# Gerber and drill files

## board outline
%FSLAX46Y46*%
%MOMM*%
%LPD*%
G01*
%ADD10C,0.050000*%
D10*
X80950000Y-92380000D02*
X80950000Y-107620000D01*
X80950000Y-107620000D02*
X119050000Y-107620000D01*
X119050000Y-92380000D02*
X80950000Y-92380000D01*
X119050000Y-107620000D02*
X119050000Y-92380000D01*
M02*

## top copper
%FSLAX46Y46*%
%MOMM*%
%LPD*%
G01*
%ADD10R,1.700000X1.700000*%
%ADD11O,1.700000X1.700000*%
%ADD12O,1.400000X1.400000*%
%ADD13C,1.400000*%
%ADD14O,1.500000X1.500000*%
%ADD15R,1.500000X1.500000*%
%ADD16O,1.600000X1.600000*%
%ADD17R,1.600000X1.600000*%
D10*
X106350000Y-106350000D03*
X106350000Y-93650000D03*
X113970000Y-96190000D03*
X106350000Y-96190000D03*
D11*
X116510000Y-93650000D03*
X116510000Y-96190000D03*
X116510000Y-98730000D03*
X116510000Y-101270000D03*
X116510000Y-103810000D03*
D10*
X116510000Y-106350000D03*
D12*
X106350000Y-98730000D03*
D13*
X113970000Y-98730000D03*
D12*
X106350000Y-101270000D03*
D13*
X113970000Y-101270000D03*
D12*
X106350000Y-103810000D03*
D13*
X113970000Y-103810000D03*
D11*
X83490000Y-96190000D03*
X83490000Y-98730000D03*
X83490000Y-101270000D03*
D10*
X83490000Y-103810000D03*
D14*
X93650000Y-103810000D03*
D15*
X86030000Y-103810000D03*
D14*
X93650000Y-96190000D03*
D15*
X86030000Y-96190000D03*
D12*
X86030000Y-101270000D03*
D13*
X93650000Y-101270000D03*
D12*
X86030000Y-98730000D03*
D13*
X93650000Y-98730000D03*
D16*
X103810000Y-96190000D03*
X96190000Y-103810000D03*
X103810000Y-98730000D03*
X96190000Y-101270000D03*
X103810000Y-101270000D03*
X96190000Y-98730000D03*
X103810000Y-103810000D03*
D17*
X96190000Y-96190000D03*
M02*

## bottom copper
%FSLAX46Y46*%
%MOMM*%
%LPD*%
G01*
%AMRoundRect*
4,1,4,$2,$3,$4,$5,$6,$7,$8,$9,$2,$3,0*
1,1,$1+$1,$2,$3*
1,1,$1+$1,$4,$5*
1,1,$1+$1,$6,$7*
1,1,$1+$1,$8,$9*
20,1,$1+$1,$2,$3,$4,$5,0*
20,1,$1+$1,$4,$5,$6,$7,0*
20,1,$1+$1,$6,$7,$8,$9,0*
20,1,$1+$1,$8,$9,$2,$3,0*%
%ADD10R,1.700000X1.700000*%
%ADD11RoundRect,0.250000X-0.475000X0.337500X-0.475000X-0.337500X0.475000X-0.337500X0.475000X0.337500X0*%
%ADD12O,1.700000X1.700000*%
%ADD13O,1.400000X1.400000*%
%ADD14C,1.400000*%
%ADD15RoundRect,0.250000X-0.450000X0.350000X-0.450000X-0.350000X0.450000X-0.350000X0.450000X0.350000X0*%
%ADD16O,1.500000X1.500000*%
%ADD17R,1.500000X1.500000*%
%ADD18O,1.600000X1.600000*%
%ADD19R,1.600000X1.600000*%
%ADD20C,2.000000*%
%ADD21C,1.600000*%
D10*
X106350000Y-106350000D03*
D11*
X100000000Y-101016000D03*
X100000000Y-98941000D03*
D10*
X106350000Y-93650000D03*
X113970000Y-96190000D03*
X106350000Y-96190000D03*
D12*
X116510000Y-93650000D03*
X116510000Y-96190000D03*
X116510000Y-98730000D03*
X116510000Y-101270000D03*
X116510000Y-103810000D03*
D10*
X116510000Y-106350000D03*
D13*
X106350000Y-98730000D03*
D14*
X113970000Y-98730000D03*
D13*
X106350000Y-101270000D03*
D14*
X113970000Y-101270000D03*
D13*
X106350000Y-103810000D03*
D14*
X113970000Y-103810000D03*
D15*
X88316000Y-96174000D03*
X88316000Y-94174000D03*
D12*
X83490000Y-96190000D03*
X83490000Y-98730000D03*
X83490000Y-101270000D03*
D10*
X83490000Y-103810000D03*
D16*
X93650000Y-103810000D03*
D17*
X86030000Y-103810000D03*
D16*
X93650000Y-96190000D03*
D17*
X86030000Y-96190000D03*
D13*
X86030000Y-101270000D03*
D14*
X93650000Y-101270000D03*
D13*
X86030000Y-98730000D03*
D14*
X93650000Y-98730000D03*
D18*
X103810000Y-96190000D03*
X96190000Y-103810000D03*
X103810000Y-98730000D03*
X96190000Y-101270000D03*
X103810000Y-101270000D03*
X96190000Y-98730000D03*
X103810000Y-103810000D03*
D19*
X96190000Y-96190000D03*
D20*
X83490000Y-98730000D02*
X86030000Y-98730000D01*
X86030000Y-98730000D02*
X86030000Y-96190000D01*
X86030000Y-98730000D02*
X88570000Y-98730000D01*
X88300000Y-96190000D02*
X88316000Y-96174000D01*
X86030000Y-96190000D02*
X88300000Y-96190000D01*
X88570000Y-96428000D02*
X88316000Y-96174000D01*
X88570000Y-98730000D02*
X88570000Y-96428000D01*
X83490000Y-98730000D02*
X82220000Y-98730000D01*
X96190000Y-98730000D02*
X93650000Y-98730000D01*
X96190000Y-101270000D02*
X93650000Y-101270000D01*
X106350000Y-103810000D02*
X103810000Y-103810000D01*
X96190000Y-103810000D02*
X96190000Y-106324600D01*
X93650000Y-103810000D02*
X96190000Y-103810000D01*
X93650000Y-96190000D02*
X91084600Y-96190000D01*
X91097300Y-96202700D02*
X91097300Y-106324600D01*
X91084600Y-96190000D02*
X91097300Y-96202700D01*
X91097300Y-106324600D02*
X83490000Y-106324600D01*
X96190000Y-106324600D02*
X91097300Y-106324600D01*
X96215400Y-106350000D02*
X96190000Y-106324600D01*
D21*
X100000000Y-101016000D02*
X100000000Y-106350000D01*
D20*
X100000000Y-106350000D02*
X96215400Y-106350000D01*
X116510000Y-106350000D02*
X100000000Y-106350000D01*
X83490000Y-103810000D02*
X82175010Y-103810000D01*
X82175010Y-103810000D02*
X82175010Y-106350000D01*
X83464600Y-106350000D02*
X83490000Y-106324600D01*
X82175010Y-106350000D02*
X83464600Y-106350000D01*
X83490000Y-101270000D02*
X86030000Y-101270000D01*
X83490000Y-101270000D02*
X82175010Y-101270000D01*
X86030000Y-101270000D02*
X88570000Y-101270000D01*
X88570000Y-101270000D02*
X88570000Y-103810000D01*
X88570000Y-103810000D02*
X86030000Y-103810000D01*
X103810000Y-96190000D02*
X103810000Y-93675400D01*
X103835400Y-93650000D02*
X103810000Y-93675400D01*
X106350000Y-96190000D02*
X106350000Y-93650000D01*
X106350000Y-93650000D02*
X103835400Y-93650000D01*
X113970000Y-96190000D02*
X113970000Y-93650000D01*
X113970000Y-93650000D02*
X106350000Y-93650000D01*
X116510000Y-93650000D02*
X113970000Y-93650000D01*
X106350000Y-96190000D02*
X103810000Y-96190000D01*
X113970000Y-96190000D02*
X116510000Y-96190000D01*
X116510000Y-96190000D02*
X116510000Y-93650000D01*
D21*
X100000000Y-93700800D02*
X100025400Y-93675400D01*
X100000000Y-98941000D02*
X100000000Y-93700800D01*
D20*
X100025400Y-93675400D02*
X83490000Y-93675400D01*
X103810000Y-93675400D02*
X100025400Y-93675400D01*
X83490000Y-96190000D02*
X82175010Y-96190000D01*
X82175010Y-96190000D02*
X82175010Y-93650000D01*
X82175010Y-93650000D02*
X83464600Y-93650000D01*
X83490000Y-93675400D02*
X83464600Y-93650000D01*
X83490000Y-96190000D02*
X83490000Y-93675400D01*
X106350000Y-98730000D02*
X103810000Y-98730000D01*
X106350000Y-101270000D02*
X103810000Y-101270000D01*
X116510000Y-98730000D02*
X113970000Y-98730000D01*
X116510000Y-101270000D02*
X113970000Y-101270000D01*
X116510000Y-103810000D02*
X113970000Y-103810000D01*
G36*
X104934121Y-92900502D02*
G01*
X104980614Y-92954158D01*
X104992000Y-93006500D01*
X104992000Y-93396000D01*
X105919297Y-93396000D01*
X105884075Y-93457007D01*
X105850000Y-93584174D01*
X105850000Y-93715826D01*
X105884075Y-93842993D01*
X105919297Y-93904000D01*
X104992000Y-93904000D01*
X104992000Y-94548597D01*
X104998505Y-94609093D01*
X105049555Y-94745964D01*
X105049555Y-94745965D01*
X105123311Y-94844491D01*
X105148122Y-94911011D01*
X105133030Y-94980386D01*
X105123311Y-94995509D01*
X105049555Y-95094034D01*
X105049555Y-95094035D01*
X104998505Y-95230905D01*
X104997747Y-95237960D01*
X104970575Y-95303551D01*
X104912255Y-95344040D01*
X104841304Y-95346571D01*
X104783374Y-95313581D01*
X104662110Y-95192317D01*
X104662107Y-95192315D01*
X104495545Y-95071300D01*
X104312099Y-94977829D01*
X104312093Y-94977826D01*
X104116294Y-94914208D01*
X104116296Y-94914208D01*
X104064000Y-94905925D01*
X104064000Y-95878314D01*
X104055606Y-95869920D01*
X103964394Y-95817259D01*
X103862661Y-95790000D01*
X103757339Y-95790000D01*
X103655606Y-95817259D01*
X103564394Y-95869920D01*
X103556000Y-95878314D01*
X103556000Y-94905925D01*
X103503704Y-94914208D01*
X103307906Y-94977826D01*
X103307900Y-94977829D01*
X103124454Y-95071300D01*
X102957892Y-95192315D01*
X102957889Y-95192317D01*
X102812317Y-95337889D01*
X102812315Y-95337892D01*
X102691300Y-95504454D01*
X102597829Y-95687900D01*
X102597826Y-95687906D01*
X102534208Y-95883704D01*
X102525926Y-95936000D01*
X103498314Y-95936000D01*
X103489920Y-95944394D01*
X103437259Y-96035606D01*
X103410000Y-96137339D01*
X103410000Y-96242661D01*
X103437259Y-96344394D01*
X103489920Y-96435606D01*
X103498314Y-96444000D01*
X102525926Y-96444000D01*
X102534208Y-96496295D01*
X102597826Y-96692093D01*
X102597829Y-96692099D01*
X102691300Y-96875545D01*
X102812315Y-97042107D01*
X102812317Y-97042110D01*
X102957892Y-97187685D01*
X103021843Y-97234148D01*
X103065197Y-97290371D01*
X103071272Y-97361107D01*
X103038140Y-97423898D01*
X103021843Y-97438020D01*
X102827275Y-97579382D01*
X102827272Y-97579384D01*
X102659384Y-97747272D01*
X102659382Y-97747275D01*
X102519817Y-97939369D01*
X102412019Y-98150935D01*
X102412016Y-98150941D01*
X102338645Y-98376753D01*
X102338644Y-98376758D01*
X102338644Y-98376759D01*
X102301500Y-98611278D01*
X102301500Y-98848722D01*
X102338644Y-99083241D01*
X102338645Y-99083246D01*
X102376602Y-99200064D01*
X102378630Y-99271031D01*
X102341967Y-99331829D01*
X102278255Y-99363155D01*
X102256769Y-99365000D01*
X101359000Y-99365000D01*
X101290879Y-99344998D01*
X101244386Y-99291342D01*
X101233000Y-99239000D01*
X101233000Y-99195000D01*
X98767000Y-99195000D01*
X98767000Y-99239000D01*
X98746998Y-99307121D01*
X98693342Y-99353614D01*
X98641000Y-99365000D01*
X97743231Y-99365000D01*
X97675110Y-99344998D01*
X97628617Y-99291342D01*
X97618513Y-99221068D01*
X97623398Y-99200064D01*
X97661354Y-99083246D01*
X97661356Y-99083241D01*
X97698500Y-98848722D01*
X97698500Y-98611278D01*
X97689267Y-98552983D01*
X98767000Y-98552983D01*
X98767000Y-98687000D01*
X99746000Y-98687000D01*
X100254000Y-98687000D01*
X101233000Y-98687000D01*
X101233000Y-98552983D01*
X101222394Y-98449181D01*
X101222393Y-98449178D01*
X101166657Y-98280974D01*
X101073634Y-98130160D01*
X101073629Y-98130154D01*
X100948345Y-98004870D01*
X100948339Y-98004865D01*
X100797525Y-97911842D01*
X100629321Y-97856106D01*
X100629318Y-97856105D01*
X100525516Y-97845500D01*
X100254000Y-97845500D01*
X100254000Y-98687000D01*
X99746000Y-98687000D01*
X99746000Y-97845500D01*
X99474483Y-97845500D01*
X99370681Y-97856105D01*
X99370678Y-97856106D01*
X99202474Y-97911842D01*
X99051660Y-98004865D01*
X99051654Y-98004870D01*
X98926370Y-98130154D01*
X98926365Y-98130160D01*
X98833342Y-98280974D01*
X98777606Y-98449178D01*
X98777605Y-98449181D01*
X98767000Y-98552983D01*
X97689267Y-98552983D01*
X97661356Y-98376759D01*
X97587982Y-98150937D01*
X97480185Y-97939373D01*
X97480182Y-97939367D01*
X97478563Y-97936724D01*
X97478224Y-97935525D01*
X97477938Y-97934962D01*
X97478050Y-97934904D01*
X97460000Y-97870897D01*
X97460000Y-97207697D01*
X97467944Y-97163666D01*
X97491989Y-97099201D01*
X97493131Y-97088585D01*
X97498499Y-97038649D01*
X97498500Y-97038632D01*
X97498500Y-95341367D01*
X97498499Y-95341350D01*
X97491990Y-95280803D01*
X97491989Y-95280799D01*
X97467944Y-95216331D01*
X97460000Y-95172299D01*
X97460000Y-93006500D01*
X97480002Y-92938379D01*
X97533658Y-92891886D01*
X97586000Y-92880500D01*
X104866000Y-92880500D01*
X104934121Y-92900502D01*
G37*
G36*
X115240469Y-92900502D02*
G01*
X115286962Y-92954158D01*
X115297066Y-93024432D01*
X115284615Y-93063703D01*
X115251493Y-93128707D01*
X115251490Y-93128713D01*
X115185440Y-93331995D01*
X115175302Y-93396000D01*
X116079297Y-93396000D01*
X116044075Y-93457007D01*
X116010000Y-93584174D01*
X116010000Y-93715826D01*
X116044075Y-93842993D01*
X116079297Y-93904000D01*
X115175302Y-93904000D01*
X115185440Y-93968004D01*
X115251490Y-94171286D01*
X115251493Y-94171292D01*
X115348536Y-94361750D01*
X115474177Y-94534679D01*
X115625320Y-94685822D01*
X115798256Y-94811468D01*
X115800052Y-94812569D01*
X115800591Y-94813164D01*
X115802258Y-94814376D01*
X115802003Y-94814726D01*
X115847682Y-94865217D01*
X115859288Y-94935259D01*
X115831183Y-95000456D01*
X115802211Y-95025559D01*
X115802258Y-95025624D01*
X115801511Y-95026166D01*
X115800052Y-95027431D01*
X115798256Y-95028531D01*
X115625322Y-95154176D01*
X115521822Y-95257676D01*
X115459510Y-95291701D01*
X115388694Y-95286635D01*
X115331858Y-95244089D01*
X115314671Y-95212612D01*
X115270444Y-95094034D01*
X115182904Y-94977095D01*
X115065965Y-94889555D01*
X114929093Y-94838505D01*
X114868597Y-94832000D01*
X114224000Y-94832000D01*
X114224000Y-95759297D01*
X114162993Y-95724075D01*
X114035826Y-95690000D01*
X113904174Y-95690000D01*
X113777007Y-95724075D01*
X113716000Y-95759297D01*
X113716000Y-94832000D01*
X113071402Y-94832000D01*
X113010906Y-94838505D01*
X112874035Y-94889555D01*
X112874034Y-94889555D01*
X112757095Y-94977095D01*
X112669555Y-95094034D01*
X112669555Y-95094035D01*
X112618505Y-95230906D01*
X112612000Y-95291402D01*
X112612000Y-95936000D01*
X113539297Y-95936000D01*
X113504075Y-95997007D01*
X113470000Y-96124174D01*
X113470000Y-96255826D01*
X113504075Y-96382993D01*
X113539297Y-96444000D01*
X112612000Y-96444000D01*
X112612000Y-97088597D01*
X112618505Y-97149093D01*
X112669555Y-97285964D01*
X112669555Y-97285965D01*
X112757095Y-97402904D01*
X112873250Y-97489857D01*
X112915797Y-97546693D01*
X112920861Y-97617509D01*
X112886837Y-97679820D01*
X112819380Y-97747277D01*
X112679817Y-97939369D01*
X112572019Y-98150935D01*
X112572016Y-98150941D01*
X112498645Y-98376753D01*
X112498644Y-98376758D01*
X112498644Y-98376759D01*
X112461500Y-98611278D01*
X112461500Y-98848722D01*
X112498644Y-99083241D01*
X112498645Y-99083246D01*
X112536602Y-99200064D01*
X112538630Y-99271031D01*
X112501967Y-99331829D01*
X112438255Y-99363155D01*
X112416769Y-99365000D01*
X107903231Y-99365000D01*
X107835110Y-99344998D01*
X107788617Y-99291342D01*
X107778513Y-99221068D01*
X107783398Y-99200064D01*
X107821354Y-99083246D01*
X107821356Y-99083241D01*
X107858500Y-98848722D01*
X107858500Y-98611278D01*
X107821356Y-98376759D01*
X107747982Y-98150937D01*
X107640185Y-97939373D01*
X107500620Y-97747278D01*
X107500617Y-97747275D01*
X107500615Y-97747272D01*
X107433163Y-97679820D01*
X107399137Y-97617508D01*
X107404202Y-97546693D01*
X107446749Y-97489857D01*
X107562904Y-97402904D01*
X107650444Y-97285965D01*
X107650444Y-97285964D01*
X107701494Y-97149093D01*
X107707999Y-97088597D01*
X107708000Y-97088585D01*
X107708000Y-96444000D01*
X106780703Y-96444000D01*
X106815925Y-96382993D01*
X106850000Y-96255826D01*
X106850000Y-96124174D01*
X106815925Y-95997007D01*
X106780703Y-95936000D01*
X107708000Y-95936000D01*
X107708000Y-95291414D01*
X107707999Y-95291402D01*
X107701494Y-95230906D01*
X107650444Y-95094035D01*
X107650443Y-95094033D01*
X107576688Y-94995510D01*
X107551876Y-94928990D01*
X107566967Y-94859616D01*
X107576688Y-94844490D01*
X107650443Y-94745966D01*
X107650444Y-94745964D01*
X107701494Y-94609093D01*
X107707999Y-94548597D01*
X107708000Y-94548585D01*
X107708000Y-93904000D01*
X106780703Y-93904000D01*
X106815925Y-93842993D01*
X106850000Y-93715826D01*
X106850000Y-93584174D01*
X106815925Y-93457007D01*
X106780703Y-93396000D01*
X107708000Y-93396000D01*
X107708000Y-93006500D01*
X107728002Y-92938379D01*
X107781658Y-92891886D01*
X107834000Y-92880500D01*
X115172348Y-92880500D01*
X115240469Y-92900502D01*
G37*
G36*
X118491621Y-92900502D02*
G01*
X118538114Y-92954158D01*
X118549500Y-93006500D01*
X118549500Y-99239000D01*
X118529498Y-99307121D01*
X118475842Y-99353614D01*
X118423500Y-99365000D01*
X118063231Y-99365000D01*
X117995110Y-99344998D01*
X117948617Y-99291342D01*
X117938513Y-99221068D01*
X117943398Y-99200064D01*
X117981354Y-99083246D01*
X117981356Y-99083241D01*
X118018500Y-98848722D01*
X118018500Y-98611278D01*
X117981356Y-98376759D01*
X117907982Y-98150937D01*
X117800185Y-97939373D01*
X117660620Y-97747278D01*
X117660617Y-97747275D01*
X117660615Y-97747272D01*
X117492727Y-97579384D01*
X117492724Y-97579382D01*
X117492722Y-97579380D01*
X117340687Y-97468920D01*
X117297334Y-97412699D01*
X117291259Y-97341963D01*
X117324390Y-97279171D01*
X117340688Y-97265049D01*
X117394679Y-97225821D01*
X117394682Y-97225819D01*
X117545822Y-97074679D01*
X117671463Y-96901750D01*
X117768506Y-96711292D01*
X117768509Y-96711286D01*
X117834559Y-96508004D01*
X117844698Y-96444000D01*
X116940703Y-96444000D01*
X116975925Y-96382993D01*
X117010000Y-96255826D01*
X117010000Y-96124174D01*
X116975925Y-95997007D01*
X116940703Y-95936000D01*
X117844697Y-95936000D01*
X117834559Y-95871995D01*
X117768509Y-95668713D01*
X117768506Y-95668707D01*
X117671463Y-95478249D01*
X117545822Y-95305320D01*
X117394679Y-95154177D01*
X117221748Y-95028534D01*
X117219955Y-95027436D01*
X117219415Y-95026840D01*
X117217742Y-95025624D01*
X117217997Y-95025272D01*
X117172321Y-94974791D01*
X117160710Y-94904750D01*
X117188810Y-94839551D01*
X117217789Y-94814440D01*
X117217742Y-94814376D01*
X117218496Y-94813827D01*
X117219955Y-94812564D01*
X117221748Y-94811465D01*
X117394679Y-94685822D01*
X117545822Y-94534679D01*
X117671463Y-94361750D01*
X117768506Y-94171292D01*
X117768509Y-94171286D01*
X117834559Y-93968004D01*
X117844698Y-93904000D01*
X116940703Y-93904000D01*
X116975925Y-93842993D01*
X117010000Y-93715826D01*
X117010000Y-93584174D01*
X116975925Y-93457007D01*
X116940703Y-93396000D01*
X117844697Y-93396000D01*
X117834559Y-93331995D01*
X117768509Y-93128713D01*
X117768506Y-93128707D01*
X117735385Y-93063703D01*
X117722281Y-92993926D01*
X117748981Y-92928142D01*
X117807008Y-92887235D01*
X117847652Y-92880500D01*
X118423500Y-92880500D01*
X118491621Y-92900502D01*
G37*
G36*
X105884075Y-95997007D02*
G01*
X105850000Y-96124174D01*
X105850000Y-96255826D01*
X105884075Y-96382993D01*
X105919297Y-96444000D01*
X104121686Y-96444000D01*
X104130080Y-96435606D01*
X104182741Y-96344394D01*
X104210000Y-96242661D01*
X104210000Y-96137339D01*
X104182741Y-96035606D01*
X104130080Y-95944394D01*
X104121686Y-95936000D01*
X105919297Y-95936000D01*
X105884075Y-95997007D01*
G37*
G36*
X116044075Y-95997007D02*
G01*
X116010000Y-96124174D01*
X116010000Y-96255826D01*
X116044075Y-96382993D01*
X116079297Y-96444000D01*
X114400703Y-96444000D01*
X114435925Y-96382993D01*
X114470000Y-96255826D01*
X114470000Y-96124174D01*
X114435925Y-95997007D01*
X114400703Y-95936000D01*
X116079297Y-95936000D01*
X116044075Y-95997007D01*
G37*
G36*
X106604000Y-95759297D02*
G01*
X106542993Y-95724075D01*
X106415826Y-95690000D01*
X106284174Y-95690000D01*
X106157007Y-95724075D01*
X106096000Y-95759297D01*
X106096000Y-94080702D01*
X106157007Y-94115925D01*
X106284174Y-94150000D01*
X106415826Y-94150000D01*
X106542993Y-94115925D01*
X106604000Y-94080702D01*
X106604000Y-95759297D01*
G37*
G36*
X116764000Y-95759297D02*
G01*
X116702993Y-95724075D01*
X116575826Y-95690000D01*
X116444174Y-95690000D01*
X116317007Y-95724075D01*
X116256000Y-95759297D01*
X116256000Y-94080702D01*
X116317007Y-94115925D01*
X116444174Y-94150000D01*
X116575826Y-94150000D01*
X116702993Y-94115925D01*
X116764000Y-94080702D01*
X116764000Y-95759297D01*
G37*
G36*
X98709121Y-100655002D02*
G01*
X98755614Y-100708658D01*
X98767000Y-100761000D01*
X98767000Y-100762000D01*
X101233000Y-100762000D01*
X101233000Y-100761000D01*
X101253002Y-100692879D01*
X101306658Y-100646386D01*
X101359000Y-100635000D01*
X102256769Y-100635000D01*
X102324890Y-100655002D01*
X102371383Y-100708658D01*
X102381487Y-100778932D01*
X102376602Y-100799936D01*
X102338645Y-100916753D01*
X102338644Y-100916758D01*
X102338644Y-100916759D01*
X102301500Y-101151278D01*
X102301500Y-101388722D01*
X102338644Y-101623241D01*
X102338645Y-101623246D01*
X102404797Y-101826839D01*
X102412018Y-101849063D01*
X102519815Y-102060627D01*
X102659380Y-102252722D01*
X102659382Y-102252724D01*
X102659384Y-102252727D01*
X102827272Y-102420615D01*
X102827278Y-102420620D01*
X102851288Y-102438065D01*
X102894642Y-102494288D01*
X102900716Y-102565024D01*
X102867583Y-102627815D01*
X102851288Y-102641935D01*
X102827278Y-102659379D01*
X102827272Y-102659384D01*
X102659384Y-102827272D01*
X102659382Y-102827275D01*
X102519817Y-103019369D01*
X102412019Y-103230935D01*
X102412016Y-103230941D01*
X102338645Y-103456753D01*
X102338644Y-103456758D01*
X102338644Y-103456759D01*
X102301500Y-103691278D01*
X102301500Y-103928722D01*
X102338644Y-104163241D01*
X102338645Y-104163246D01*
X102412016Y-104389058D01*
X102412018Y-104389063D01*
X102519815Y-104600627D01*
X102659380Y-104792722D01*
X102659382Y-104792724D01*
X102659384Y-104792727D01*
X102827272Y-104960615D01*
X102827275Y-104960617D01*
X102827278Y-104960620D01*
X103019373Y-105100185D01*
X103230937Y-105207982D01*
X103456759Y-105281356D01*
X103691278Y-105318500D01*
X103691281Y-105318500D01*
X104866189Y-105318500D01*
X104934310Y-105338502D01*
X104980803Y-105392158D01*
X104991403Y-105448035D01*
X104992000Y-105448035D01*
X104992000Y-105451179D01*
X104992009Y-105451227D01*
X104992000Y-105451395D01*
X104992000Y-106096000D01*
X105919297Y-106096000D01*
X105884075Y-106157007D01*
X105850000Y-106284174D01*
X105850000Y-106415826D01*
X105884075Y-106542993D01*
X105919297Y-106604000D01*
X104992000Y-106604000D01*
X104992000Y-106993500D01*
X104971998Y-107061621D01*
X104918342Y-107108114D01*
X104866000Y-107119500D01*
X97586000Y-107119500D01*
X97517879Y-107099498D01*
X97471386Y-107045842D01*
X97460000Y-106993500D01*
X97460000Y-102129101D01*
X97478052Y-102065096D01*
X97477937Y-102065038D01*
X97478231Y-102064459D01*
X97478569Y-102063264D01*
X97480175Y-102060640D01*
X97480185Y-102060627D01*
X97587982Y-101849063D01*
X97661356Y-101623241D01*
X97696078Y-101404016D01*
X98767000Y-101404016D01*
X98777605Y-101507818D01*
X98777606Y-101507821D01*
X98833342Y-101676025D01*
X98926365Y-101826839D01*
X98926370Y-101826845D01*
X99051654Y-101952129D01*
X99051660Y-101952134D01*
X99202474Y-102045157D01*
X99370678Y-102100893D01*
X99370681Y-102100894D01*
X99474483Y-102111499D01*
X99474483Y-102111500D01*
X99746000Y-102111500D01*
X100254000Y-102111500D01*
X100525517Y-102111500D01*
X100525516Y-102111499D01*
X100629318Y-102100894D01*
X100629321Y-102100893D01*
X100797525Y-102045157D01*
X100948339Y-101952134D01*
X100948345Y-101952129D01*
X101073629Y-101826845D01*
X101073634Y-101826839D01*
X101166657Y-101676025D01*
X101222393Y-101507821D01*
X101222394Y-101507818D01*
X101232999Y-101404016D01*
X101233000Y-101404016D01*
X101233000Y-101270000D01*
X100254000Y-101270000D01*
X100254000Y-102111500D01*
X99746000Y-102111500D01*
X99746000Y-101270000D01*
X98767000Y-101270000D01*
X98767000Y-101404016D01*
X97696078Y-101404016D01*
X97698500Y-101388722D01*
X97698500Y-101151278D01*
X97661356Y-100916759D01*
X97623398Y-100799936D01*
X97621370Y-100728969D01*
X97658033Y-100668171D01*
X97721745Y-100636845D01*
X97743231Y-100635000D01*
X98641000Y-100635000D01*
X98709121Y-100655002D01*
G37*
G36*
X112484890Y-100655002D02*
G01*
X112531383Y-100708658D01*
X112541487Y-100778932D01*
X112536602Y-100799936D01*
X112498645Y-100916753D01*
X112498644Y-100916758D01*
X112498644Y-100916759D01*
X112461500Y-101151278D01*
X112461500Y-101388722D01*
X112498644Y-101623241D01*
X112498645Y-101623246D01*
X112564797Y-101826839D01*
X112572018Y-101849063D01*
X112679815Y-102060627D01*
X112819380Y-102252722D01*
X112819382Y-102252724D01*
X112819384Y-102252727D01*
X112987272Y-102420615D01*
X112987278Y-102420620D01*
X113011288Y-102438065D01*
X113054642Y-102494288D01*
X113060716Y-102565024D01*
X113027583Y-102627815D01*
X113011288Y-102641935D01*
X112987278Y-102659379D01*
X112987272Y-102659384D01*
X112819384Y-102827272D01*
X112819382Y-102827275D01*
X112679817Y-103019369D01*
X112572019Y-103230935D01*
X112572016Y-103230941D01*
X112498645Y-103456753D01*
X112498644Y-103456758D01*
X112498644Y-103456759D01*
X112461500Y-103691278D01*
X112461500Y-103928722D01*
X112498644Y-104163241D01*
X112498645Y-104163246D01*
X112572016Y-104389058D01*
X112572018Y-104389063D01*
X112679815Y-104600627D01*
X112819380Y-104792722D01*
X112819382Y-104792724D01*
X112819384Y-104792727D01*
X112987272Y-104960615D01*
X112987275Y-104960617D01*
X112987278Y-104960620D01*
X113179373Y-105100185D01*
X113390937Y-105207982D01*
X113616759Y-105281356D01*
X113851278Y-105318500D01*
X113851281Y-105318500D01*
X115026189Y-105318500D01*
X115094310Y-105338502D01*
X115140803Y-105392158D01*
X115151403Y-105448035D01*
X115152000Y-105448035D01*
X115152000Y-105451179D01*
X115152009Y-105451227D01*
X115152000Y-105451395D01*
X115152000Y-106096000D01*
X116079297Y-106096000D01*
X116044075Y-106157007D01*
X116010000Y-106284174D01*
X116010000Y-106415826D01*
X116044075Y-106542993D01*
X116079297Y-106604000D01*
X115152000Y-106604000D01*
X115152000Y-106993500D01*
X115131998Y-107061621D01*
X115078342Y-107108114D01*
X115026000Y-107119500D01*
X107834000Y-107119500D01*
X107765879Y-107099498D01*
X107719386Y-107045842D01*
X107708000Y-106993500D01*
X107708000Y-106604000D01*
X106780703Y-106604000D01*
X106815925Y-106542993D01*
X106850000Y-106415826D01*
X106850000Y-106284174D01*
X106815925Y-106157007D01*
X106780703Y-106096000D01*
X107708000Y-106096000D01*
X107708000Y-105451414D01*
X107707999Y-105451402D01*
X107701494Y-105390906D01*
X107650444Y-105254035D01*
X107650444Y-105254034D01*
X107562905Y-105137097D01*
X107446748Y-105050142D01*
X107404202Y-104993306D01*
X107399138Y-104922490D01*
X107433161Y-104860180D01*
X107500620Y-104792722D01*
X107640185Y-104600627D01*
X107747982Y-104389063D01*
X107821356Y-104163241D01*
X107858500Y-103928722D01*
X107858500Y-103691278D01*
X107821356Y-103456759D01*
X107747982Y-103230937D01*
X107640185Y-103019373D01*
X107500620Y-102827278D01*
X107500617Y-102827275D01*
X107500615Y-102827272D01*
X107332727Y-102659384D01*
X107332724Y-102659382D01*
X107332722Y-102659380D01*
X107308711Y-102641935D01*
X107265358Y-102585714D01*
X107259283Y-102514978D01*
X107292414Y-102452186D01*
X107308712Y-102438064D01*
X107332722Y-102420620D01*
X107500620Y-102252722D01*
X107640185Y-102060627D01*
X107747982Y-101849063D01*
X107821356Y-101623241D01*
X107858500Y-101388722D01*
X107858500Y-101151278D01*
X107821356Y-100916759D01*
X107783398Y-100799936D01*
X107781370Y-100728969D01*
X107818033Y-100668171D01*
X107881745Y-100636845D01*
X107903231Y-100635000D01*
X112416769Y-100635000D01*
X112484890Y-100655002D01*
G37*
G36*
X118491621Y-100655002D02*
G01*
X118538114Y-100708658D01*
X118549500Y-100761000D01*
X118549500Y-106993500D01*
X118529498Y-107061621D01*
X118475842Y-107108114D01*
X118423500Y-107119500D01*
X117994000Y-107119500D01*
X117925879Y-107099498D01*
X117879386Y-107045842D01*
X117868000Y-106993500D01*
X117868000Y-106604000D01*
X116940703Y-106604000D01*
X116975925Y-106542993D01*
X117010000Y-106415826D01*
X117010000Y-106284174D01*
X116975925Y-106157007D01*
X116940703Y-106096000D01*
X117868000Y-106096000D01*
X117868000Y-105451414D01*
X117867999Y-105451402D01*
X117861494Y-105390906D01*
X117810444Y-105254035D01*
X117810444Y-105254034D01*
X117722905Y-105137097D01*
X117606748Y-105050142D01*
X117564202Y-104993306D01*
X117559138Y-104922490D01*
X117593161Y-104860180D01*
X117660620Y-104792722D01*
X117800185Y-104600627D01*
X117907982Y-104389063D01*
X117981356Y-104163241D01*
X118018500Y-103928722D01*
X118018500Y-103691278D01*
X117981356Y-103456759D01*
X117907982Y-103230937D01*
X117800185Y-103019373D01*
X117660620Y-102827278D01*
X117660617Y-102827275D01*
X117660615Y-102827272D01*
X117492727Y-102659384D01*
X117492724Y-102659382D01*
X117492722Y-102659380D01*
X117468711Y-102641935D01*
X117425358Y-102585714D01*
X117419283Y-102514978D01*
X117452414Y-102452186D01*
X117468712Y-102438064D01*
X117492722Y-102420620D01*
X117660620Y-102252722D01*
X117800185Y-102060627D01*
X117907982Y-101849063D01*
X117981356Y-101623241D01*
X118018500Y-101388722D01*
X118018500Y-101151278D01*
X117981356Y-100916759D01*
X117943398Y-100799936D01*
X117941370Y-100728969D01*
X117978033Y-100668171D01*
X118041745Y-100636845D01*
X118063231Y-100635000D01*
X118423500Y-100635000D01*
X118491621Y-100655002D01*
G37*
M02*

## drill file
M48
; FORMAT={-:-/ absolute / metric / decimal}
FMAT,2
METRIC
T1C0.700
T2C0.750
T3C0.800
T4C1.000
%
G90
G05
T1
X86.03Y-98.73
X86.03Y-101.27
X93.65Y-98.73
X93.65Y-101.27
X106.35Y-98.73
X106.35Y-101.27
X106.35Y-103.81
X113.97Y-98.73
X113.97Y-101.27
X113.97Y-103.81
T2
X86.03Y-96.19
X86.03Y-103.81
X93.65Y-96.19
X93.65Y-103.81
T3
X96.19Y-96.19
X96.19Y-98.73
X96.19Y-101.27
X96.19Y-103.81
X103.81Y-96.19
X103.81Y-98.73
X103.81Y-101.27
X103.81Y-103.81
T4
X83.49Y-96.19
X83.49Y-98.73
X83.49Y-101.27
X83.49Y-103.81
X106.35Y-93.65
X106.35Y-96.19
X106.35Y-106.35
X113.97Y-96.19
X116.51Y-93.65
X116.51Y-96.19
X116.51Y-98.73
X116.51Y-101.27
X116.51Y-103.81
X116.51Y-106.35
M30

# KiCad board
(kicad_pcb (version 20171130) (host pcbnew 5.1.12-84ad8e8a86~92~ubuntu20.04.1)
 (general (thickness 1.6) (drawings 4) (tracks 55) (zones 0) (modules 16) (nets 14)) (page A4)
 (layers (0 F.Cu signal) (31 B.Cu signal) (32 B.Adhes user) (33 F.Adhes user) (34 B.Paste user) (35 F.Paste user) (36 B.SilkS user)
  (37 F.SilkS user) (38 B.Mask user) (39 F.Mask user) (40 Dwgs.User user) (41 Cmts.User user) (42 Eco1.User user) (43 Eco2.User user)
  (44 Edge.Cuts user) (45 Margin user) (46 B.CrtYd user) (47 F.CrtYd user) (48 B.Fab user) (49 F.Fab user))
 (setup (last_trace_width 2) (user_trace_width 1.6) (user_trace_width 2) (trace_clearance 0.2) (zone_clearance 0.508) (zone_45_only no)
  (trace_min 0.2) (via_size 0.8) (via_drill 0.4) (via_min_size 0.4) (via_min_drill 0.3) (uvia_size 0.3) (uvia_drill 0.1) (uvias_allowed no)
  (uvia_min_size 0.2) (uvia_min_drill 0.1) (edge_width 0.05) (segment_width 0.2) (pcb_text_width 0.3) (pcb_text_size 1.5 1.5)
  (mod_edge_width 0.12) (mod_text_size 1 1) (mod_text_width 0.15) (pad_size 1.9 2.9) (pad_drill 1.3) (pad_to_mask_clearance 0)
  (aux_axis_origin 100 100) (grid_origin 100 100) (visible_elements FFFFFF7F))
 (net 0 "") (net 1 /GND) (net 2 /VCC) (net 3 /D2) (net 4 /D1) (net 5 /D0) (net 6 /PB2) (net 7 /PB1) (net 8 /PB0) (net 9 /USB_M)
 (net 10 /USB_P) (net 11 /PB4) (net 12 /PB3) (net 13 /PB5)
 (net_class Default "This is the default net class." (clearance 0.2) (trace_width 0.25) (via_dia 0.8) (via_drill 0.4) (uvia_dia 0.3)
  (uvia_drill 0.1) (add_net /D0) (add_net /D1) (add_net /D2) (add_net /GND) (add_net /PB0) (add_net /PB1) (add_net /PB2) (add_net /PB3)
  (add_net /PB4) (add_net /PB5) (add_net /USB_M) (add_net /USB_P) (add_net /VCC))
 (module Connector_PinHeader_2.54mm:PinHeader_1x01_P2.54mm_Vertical (layer F.Cu) (at 106.35 106.35)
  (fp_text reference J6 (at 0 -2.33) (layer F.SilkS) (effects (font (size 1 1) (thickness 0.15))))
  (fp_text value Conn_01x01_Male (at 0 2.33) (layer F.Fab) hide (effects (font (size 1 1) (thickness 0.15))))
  (pad 1 thru_hole rect (at 0 0) (size 1.7 1.7) (drill 1) (layers *.Cu *.Mask) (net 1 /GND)))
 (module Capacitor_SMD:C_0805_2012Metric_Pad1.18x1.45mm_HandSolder (layer B.Cu) (at 100 99.9785 270)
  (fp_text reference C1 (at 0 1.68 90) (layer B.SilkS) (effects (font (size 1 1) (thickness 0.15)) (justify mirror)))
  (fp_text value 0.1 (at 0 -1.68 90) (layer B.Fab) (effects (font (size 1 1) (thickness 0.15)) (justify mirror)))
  (pad 2 smd roundrect (at 1.0375 0 270) (size 1.175 1.45) (layers B.Cu B.Paste B.Mask) (roundrect_rratio 0.212766) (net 1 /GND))
  (pad 1 smd roundrect (at -1.0375 0 270) (size 1.175 1.45) (layers B.Cu B.Paste B.Mask) (roundrect_rratio 0.212766) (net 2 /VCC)))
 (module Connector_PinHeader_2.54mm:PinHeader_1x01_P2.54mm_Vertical (layer F.Cu) (at 106.35 93.65)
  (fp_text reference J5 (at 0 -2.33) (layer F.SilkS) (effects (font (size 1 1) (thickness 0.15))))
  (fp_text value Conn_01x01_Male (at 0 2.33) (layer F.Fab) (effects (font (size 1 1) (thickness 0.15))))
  (pad 1 thru_hole rect (at 0 0) (size 1.7 1.7) (drill 1) (layers *.Cu *.Mask) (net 2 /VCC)))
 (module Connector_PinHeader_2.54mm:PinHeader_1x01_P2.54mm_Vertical (layer F.Cu) (at 113.97 96.19)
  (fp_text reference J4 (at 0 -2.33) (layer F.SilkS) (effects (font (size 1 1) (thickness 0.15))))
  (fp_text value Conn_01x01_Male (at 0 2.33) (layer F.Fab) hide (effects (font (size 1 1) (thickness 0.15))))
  (pad 1 thru_hole rect (at 0 0) (size 1.7 1.7) (drill 1) (layers *.Cu *.Mask) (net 2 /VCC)))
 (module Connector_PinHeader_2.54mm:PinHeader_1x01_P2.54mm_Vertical (layer F.Cu) (at 106.35 96.19)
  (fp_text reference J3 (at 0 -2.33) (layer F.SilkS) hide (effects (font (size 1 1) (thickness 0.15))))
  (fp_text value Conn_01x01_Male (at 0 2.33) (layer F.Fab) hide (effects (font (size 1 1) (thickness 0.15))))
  (pad 1 thru_hole rect (at 0 0) (size 1.7 1.7) (drill 1) (layers *.Cu *.Mask) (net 2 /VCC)))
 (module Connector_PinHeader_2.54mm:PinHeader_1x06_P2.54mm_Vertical (layer F.Cu) (at 116.51 106.35 180)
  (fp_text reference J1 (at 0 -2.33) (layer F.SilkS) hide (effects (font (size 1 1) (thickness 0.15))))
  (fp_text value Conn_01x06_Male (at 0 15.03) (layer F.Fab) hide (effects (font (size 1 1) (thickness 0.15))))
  (pad 6 thru_hole oval (at 0 12.7 180) (size 1.7 1.7) (drill 1) (layers *.Cu *.Mask) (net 2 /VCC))
  (pad 5 thru_hole oval (at 0 10.16 180) (size 1.7 1.7) (drill 1) (layers *.Cu *.Mask) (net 2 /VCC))
  (pad 4 thru_hole oval (at 0 7.62 180) (size 1.7 1.7) (drill 1) (layers *.Cu *.Mask) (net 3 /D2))
  (pad 3 thru_hole oval (at 0 5.08 180) (size 1.7 1.7) (drill 1) (layers *.Cu *.Mask) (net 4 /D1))
  (pad 2 thru_hole oval (at 0 2.54 180) (size 1.7 1.7) (drill 1) (layers *.Cu *.Mask) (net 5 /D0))
  (pad 1 thru_hole rect (at 0 0 180) (size 1.7 1.7) (drill 1) (layers *.Cu *.Mask) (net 1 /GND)))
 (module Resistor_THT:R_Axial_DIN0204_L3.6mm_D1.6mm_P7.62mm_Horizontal (layer F.Cu) (at 113.97 98.73 180)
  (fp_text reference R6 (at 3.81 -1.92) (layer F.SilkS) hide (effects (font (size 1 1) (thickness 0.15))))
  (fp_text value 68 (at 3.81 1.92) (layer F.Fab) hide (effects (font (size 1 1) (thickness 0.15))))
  (pad 2 thru_hole oval (at 7.62 0 180) (size 1.4 1.4) (drill 0.7) (layers *.Cu *.Mask) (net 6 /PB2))
  (pad 1 thru_hole circle (at 0 0 180) (size 1.4 1.4) (drill 0.7) (layers *.Cu *.Mask) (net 3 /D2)))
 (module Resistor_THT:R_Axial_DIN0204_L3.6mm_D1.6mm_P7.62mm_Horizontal (layer F.Cu) (at 113.97 101.27 180)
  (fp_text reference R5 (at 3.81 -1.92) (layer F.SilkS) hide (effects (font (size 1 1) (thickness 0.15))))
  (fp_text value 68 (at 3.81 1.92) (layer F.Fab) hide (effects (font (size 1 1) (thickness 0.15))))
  (pad 2 thru_hole oval (at 7.62 0 180) (size 1.4 1.4) (drill 0.7) (layers *.Cu *.Mask) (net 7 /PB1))
  (pad 1 thru_hole circle (at 0 0 180) (size 1.4 1.4) (drill 0.7) (layers *.Cu *.Mask) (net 4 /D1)))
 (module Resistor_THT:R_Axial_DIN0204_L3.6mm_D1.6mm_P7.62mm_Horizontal (layer F.Cu) (at 113.97 103.81 180)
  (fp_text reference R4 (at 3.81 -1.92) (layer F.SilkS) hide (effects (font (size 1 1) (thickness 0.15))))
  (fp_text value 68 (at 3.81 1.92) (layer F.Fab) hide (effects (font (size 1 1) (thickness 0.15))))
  (pad 2 thru_hole oval (at 7.62 0 180) (size 1.4 1.4) (drill 0.7) (layers *.Cu *.Mask) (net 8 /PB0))
  (pad 1 thru_hole circle (at 0 0 180) (size 1.4 1.4) (drill 0.7) (layers *.Cu *.Mask) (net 5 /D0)))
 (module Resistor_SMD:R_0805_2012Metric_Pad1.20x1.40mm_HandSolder (layer B.Cu) (at 88.316 95.174 270)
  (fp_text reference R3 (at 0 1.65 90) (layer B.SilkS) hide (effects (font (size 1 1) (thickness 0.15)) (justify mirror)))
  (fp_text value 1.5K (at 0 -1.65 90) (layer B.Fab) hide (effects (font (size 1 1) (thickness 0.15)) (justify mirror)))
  (pad 2 smd roundrect (at 1 0 270) (size 1.2 1.4) (layers B.Cu B.Paste B.Mask) (roundrect_rratio 0.208333) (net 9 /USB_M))
  (pad 1 smd roundrect (at -1 0 270) (size 1.2 1.4) (layers B.Cu B.Paste B.Mask) (roundrect_rratio 0.208333) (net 2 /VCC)))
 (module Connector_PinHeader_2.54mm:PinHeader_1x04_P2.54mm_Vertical (layer F.Cu) (at 83.49 103.81 180)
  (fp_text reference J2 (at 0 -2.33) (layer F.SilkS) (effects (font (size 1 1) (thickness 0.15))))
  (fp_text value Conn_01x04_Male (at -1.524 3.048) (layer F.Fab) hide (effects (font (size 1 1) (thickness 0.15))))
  (pad 4 thru_hole oval (at 0 7.62 180) (size 1.7 1.7) (drill 1) (layers *.Cu *.Mask) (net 2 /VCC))
  (pad 3 thru_hole oval (at 0 5.08 180) (size 1.7 1.7) (drill 1) (layers *.Cu *.Mask) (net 9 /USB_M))
  (pad 2 thru_hole oval (at 0 2.54 180) (size 1.7 1.7) (drill 1) (layers *.Cu *.Mask) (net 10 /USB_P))
  (pad 1 thru_hole rect (at 0 0 180) (size 1.7 1.7) (drill 1) (layers *.Cu *.Mask) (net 1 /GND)))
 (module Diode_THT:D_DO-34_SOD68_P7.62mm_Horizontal (layer F.Cu) (at 86.03 103.81)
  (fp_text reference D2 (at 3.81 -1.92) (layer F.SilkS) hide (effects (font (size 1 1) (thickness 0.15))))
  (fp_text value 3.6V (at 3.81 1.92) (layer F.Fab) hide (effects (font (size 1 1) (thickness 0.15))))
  (pad 2 thru_hole oval (at 7.62 0) (size 1.5 1.5) (drill 0.75) (layers *.Cu *.Mask) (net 1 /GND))
  (pad 1 thru_hole rect (at 0 0) (size 1.5 1.5) (drill 0.75) (layers *.Cu *.Mask) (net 10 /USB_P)))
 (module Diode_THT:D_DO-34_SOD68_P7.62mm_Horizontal (layer F.Cu) (at 86.03 96.19)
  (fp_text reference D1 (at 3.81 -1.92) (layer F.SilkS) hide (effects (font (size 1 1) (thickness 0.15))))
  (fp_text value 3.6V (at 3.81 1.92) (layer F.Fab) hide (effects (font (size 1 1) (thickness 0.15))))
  (pad 2 thru_hole oval (at 7.62 0) (size 1.5 1.5) (drill 0.75) (layers *.Cu *.Mask) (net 1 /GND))
  (pad 1 thru_hole rect (at 0 0) (size 1.5 1.5) (drill 0.75) (layers *.Cu *.Mask) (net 9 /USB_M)))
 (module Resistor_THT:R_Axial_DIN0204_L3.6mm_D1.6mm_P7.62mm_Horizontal (layer F.Cu) (at 93.65 101.27 180)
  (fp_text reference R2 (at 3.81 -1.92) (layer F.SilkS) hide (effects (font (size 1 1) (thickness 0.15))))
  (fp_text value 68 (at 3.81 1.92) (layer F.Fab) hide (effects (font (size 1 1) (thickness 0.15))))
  (pad 2 thru_hole oval (at 7.62 0 180) (size 1.4 1.4) (drill 0.7) (layers *.Cu *.Mask) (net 10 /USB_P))
  (pad 1 thru_hole circle (at 0 0 180) (size 1.4 1.4) (drill 0.7) (layers *.Cu *.Mask) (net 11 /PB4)))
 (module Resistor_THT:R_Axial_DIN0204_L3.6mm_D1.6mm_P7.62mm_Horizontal (layer F.Cu) (at 93.65 98.73 180)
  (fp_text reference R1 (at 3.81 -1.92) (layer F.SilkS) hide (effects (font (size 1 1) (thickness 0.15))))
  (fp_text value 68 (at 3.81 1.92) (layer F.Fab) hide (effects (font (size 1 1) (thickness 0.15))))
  (pad 2 thru_hole oval (at 7.62 0 180) (size 1.4 1.4) (drill 0.7) (layers *.Cu *.Mask) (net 9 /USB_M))
  (pad 1 thru_hole circle (at 0 0 180) (size 1.4 1.4) (drill 0.7) (layers *.Cu *.Mask) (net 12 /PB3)))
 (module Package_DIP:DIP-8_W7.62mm (layer F.Cu) (at 96.19 96.19)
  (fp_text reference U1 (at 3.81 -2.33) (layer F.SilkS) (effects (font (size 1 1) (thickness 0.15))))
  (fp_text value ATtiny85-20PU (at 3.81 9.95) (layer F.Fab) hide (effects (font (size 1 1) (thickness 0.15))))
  (pad 8 thru_hole oval (at 7.62 0) (size 1.6 1.6) (drill 0.8) (layers *.Cu *.Mask) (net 2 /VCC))
  (pad 4 thru_hole oval (at 0 7.62) (size 1.6 1.6) (drill 0.8) (layers *.Cu *.Mask) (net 1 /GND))
  (pad 7 thru_hole oval (at 7.62 2.54) (size 1.6 1.6) (drill 0.8) (layers *.Cu *.Mask) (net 6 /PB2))
  (pad 3 thru_hole oval (at 0 5.08) (size 1.6 1.6) (drill 0.8) (layers *.Cu *.Mask) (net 11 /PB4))
  (pad 6 thru_hole oval (at 7.62 5.08) (size 1.6 1.6) (drill 0.8) (layers *.Cu *.Mask) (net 7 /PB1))
  (pad 2 thru_hole oval (at 0 2.54) (size 1.6 1.6) (drill 0.8) (layers *.Cu *.Mask) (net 12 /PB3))
  (pad 5 thru_hole oval (at 7.62 7.62) (size 1.6 1.6) (drill 0.8) (layers *.Cu *.Mask) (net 8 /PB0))
  (pad 1 thru_hole rect (at 0 0) (size 1.6 1.6) (drill 0.8) (layers *.Cu *.Mask) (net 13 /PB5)))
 (gr_line (start 80.95 92.38) (end 80.95 107.62) (layer Edge.Cuts) (width 0.05))
 (gr_line (start 80.95 107.62) (end 119.05 107.62) (layer Edge.Cuts) (width 0.05))
 (gr_line (start 119.05 92.38) (end 80.95 92.38) (layer Edge.Cuts) (width 0.05))
 (gr_line (start 119.05 107.62) (end 119.05 92.38) (layer Edge.Cuts) (width 0.05))
 (segment (start 83.49 98.73) (end 86.03 98.73) (width 2) (layer B.Cu) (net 9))
 (segment (start 86.03 98.73) (end 86.03 96.19) (width 2) (layer B.Cu) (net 9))
 (segment (start 86.03 98.73) (end 88.57 98.73) (width 2) (layer B.Cu) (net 9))
 (segment (start 88.3 96.19) (end 88.316 96.174) (width 2) (layer B.Cu) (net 9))
 (segment (start 86.03 96.19) (end 88.3 96.19) (width 2) (layer B.Cu) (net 9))
 (segment (start 88.57 96.428) (end 88.316 96.174) (width 2) (layer B.Cu) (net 9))
 (segment (start 88.57 98.73) (end 88.57 96.428) (width 2) (layer B.Cu) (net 9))
 (segment (start 83.49 98.73) (end 82.22 98.73) (width 2) (layer B.Cu) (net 9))
 (segment (start 96.19 98.73) (end 93.65 98.73) (width 2) (layer B.Cu) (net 12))
 (segment (start 96.19 101.27) (end 93.65 101.27) (width 2) (layer B.Cu) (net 11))
 (segment (start 106.35 103.81) (end 103.81 103.81) (width 2) (layer B.Cu) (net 8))
 (segment (start 96.19 103.81) (end 96.19 106.3246) (width 2) (layer B.Cu) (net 1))
 (segment (start 93.65 103.81) (end 96.19 103.81) (width 2) (layer B.Cu) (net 1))
 (segment (start 93.65 96.19) (end 91.0846 96.19) (width 2) (layer B.Cu) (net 1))
 (segment (start 91.0973 96.2027) (end 91.0973 106.3246) (width 2) (layer B.Cu) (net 1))
 (segment (start 91.0846 96.19) (end 91.0973 96.2027) (width 2) (layer B.Cu) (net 1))
 (segment (start 91.0973 106.3246) (end 83.49 106.3246) (width 2) (layer B.Cu) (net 1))
 (segment (start 96.19 106.3246) (end 91.0973 106.3246) (width 2) (layer B.Cu) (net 1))
 (segment (start 96.2154 106.35) (end 96.19 106.3246) (width 2) (layer B.Cu) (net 1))
 (segment (start 100 101.016) (end 100 106.35) (width 1.6) (layer B.Cu) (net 1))
 (segment (start 100 106.35) (end 96.2154 106.35) (width 2) (layer B.Cu) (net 1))
 (segment (start 116.51 106.35) (end 100 106.35) (width 2) (layer B.Cu) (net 1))
 (segment (start 83.49 103.81) (end 82.17501 103.81) (width 2) (layer B.Cu) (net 1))
 (segment (start 82.17501 103.81) (end 82.17501 106.35) (width 2) (layer B.Cu) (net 1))
 (segment (start 83.4646 106.35) (end 83.49 106.3246) (width 2) (layer B.Cu) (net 1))
 (segment (start 82.17501 106.35) (end 83.4646 106.35) (width 2) (layer B.Cu) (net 1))
 (segment (start 83.49 101.27) (end 86.03 101.27) (width 2) (layer B.Cu) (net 10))
 (segment (start 83.49 101.27) (end 82.17501 101.27) (width 2) (layer B.Cu) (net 10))
 (segment (start 86.03 101.27) (end 88.57 101.27) (width 2) (layer B.Cu) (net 10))
 (segment (start 88.57 101.27) (end 88.57 103.81) (width 2) (layer B.Cu) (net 10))
 (segment (start 88.57 103.81) (end 86.03 103.81) (width 2) (layer B.Cu) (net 10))
 (segment (start 103.81 96.19) (end 103.81 93.6754) (width 2) (layer B.Cu) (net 2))
 (segment (start 103.8354 93.65) (end 103.81 93.6754) (width 2) (layer B.Cu) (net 2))
 (segment (start 106.35 96.19) (end 106.35 93.65) (width 2) (layer B.Cu) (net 2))
 (segment (start 106.35 93.65) (end 103.8354 93.65) (width 2) (layer B.Cu) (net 2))
 (segment (start 113.97 96.19) (end 113.97 93.65) (width 2) (layer B.Cu) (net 2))
 (segment (start 113.97 93.65) (end 106.35 93.65) (width 2) (layer B.Cu) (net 2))
 (segment (start 116.51 93.65) (end 113.97 93.65) (width 2) (layer B.Cu) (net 2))
 (segment (start 106.35 96.19) (end 103.81 96.19) (width 2) (layer B.Cu) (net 2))
 (segment (start 113.97 96.19) (end 116.51 96.19) (width 2) (layer B.Cu) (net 2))
 (segment (start 116.51 96.19) (end 116.51 93.65) (width 2) (layer B.Cu) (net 2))
 (segment (start 100 93.7008) (end 100.0254 93.6754) (width 1.6) (layer B.Cu) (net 2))
 (segment (start 100 98.941) (end 100 93.7008) (width 1.6) (layer B.Cu) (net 2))
 (segment (start 100.0254 93.6754) (end 83.49 93.6754) (width 2) (layer B.Cu) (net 2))
 (segment (start 103.81 93.6754) (end 100.0254 93.6754) (width 2) (layer B.Cu) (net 2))
 (segment (start 83.49 96.19) (end 82.17501 96.19) (width 2) (layer B.Cu) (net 2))
 (segment (start 82.17501 96.19) (end 82.17501 93.65) (width 2) (layer B.Cu) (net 2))
 (segment (start 82.17501 93.65) (end 83.4646 93.65) (width 2) (layer B.Cu) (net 2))
 (segment (start 83.49 93.6754) (end 83.4646 93.65) (width 2) (layer B.Cu) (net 2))
 (segment (start 83.49 96.19) (end 83.49 93.6754) (width 2) (layer B.Cu) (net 2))
 (segment (start 106.35 98.73) (end 103.81 98.73) (width 2) (layer B.Cu) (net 6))
 (segment (start 106.35 101.27) (end 103.81 101.27) (width 2) (layer B.Cu) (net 7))
 (segment (start 116.51 98.73) (end 113.97 98.73) (width 2) (layer B.Cu) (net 3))
 (segment (start 116.51 101.27) (end 113.97 101.27) (width 2) (layer B.Cu) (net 4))
 (segment (start 116.51 103.81) (end 113.97 103.81) (width 2) (layer B.Cu) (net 5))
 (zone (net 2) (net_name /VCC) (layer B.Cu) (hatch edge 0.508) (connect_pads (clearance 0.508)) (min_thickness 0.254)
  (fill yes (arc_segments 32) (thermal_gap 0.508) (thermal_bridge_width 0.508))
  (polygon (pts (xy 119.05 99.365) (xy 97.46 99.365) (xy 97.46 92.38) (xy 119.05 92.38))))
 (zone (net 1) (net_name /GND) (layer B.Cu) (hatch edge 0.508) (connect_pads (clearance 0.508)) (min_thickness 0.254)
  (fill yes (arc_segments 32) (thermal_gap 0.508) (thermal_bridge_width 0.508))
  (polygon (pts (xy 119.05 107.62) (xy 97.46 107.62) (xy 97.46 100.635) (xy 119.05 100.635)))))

